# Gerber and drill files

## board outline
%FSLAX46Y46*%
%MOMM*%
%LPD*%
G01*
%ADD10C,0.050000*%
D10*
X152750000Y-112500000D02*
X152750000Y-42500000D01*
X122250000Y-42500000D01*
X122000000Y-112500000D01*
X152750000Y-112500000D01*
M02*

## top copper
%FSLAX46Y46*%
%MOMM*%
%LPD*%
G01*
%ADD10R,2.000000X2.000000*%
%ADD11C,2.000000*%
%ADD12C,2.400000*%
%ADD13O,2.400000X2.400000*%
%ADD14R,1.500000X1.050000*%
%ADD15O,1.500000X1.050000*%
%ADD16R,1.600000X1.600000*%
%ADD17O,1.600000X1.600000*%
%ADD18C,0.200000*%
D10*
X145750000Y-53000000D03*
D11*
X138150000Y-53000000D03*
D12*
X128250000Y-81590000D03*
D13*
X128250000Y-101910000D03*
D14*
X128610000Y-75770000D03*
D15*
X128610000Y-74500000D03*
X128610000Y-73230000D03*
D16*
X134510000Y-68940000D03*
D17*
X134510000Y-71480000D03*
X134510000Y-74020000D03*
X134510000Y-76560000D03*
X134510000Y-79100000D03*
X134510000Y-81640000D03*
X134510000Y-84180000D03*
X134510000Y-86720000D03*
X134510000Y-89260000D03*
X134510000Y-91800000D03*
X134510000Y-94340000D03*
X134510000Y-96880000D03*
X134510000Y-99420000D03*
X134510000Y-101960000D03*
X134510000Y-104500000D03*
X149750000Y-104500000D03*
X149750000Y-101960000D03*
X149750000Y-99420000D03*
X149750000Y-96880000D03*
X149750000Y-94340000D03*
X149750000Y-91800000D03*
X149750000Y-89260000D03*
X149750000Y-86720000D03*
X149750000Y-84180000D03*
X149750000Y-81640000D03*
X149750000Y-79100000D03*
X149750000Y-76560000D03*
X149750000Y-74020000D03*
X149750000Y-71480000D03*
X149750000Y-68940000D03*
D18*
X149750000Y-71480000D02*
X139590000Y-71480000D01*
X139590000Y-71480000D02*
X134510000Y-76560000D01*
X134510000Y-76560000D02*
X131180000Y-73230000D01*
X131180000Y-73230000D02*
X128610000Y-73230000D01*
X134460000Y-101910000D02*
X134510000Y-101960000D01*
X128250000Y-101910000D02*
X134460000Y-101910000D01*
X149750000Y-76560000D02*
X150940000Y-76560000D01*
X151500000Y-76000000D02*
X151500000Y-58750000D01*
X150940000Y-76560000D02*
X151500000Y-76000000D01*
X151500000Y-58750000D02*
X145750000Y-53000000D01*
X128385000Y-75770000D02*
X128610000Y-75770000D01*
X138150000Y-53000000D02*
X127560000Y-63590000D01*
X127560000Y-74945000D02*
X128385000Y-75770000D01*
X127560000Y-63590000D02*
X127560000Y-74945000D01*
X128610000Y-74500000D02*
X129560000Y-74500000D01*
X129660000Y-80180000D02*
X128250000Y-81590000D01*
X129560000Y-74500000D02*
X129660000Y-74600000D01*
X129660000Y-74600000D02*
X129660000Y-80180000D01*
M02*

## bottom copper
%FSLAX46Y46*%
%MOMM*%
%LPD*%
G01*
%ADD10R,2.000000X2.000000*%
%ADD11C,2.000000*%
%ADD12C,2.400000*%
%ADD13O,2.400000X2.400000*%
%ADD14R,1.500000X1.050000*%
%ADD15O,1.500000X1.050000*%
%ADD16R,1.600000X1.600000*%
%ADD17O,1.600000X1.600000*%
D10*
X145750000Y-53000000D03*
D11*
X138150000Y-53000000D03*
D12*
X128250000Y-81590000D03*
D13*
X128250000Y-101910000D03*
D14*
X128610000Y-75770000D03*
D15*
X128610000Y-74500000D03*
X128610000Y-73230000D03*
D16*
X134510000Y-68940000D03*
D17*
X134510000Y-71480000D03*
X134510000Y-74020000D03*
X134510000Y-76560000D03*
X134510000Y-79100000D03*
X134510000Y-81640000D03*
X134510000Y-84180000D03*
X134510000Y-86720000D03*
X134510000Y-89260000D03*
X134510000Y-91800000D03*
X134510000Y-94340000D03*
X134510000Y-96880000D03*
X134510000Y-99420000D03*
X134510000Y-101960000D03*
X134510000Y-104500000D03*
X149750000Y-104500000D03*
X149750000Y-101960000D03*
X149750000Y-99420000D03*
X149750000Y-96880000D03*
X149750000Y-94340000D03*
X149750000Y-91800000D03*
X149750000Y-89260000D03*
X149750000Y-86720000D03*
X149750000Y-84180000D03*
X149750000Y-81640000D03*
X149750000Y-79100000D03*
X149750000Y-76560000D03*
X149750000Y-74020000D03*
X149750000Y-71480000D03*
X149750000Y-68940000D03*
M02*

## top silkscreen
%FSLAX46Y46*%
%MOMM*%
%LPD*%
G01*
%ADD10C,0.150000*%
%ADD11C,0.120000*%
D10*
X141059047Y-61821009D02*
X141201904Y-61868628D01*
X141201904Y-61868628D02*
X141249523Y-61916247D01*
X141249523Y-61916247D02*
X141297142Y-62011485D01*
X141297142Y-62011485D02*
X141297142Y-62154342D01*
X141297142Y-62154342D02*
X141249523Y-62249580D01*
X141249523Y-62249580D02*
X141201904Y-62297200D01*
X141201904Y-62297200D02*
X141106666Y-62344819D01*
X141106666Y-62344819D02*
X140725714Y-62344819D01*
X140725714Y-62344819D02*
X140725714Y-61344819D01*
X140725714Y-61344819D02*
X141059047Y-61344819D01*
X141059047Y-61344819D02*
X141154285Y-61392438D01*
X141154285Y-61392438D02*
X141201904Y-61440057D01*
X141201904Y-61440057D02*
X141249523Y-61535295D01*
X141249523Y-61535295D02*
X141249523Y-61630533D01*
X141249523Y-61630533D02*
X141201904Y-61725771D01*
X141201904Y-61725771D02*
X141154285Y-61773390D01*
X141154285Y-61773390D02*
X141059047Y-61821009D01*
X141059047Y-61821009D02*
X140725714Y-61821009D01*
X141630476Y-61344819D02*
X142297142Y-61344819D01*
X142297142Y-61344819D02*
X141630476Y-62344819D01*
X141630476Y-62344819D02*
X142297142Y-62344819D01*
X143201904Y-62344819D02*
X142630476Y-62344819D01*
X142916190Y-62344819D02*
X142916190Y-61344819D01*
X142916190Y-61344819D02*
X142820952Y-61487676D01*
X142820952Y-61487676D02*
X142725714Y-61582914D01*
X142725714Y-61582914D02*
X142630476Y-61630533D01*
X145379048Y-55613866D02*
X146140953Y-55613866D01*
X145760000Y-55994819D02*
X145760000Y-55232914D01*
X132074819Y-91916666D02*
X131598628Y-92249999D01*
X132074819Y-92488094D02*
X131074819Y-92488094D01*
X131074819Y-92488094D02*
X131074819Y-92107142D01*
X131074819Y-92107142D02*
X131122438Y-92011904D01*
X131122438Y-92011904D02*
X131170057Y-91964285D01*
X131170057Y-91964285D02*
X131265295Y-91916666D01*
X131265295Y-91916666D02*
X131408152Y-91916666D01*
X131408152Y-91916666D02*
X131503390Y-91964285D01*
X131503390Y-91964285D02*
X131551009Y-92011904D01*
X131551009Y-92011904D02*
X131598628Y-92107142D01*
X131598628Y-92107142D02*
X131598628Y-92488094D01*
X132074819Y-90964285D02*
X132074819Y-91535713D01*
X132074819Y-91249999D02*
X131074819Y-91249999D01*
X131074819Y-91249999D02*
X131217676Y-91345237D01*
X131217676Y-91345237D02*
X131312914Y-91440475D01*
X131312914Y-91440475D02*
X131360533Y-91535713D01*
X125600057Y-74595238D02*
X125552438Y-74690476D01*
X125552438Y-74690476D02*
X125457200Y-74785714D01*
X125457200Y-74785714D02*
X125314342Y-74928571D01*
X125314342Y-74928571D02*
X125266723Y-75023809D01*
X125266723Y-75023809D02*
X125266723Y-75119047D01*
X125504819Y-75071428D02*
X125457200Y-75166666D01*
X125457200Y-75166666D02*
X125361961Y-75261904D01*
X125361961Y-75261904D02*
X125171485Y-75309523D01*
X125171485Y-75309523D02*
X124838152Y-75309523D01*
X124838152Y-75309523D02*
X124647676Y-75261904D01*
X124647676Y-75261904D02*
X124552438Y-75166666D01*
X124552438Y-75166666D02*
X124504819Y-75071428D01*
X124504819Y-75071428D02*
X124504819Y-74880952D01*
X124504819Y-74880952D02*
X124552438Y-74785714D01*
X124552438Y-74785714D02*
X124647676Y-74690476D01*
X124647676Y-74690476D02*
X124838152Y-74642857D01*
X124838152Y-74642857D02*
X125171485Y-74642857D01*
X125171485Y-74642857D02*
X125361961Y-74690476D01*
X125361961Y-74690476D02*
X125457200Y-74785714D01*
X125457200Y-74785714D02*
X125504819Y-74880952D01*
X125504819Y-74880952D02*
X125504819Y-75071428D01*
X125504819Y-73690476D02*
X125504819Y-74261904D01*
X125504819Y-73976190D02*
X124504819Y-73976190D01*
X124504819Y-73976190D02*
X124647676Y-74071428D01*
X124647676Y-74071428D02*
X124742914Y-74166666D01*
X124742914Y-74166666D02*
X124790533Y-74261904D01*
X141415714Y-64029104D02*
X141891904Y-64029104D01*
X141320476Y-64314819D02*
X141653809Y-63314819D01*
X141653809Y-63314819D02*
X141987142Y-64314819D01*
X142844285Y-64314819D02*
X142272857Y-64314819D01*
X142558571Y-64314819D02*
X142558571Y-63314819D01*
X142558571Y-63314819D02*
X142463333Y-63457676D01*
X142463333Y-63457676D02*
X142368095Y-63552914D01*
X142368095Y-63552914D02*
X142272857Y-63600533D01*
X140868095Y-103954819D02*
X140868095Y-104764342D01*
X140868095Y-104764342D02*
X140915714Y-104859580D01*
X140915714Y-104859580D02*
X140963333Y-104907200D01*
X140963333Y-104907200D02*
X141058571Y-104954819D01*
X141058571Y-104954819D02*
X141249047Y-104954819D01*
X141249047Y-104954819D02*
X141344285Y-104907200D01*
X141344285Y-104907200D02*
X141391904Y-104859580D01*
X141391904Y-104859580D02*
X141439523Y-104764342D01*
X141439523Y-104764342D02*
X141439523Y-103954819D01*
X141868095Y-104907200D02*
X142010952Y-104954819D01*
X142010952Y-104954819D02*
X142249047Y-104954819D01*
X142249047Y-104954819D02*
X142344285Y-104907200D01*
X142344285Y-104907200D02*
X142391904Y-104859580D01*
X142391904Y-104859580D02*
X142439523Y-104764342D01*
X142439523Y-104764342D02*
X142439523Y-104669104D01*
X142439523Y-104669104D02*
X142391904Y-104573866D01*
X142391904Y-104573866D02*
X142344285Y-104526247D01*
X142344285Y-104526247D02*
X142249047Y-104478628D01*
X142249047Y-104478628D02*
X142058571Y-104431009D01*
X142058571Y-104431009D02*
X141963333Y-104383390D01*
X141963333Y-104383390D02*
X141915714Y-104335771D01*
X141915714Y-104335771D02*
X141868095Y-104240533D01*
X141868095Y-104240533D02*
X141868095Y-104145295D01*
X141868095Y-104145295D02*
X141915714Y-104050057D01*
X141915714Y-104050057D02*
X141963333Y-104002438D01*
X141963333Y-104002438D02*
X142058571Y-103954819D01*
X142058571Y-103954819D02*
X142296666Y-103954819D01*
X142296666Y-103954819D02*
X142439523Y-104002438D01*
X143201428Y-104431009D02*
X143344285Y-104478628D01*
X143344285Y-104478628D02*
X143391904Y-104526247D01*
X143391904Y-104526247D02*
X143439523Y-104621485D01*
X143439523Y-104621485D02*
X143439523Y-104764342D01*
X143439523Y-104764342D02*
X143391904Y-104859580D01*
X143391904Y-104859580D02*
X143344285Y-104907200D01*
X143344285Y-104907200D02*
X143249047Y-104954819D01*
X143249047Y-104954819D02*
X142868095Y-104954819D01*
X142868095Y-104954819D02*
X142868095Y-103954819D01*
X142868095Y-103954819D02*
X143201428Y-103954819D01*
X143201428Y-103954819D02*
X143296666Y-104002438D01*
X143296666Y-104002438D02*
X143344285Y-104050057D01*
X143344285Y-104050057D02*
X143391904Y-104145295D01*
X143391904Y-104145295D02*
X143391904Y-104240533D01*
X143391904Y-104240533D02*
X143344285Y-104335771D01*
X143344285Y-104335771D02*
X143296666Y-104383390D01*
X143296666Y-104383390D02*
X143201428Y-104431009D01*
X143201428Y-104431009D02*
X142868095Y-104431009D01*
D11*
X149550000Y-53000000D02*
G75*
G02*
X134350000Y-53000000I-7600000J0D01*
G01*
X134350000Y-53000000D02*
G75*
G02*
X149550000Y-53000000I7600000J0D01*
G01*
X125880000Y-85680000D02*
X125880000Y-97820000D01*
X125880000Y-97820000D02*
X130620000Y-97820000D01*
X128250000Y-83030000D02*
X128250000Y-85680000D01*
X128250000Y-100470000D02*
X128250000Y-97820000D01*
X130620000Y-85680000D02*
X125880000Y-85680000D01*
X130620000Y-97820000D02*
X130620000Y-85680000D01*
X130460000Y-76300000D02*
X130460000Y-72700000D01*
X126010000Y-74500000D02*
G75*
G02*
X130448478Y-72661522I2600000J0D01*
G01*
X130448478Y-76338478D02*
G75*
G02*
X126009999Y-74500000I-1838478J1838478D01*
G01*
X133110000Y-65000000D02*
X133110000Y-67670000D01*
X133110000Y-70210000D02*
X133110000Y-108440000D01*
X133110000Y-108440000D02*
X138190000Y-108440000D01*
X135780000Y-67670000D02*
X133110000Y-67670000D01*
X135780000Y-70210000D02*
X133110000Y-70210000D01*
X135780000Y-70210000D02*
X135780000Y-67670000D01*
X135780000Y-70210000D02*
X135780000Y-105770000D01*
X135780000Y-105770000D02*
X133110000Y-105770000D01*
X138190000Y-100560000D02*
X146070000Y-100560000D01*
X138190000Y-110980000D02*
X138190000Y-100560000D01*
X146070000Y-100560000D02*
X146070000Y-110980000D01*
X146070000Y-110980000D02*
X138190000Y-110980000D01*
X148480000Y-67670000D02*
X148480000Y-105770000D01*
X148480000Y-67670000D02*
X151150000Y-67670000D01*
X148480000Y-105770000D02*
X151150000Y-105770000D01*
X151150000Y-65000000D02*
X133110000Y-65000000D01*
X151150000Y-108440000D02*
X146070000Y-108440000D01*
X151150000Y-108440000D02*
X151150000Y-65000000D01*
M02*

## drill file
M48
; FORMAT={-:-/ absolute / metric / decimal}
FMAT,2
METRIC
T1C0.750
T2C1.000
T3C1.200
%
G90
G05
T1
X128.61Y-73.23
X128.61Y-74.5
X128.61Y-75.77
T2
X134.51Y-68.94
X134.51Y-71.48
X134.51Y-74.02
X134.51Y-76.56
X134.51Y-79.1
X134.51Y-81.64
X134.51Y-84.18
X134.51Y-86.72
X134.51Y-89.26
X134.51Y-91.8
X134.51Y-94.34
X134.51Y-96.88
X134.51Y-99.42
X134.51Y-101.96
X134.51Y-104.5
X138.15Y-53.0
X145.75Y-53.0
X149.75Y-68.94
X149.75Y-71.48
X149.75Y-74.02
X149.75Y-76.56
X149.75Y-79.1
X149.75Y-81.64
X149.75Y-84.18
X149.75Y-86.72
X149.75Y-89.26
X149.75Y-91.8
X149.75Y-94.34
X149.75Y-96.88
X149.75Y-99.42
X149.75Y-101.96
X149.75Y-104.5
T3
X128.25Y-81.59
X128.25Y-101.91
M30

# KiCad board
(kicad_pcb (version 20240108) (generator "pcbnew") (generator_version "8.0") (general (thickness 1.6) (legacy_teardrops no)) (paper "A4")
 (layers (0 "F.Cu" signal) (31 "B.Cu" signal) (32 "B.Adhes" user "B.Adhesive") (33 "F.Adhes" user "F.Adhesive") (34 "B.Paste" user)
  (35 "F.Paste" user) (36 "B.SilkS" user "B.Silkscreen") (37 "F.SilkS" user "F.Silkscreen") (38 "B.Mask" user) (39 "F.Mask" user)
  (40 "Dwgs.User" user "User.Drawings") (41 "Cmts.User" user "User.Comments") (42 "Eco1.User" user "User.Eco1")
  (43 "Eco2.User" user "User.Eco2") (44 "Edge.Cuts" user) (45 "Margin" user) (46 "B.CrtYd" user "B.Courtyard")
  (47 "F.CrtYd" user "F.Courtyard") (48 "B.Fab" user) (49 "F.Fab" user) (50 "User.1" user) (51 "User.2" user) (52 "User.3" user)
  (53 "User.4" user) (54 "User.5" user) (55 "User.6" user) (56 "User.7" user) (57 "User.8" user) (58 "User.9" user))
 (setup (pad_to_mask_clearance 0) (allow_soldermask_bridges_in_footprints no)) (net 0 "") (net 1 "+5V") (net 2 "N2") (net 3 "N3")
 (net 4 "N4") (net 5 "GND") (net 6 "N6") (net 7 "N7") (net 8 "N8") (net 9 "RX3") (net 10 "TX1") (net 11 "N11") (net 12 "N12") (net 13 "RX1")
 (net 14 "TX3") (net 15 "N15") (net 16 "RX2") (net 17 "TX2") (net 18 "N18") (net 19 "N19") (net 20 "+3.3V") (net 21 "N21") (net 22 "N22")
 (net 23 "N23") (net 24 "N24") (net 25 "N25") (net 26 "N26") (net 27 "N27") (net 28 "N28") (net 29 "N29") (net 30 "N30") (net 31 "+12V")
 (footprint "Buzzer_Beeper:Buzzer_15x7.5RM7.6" (layer "F.Cu") (at 145.75 53 180)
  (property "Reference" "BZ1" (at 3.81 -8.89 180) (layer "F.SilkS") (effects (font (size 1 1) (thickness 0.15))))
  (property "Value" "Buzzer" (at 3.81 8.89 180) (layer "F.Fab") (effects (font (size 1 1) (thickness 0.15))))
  (fp_circle (center 3.8 0) (end 11.4 0) (stroke (width 0.12) (type solid)) (fill none) (layer "F.SilkS"))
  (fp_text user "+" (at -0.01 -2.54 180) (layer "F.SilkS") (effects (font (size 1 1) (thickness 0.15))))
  (pad "1" thru_hole rect (at 0 0 180) (size 2 2) (drill 1) (layers "*.Cu" "*.Mask") (remove_unused_layers no) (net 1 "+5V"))
  (pad "2" thru_hole circle (at 7.6 0 180) (size 2 2) (drill 1) (layers "*.Cu" "*.Mask") (remove_unused_layers no) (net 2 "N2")))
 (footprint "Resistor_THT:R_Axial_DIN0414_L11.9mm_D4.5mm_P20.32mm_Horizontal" (layer "F.Cu") (at 128.25 81.59 -90)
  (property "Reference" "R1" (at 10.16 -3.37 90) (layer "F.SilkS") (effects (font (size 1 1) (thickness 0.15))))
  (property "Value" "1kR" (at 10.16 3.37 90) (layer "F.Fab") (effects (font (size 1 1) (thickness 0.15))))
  (fp_line (start 4.09 2.37) (end 16.23 2.37) (stroke (width 0.12) (type solid)) (layer "F.SilkS"))
  (fp_line (start 16.23 2.37) (end 16.23 -2.37) (stroke (width 0.12) (type solid)) (layer "F.SilkS"))
  (fp_line (start 1.44 0) (end 4.09 0) (stroke (width 0.12) (type solid)) (layer "F.SilkS"))
  (fp_line (start 18.88 0) (end 16.23 0) (stroke (width 0.12) (type solid)) (layer "F.SilkS"))
  (fp_line (start 4.09 -2.37) (end 4.09 2.37) (stroke (width 0.12) (type solid)) (layer "F.SilkS"))
  (fp_line (start 16.23 -2.37) (end 4.09 -2.37) (stroke (width 0.12) (type solid)) (layer "F.SilkS"))
  (pad "1" thru_hole circle (at 0 0 270) (size 2.4 2.4) (drill 1.2) (layers "*.Cu" "*.Mask") (remove_unused_layers no) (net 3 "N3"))
  (pad "2" thru_hole oval (at 20.32 0 270) (size 2.4 2.4) (drill 1.2) (layers "*.Cu" "*.Mask") (remove_unused_layers no) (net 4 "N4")))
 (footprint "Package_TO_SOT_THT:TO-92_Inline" (layer "F.Cu") (at 128.61 75.77 90)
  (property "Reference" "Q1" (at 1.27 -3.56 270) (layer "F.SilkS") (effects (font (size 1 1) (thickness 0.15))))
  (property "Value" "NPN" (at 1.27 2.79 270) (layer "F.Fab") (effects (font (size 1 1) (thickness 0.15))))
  (fp_line (start -0.53 1.85) (end 3.07 1.85) (stroke (width 0.12) (type solid)) (layer "F.SilkS"))
  (fp_arc (start 1.27 -2.6) (mid 3.672087 -0.994977) (end 3.108478 1.838478) (stroke (width 0.12) (type solid)) (layer "F.SilkS"))
  (fp_arc (start -0.568478 1.838478) (mid -1.132087 -0.994977) (end 1.27 -2.6) (stroke (width 0.12) (type solid)) (layer "F.SilkS"))
  (pad "1" thru_hole rect (at 0 0 90) (size 1.05 1.5) (drill 0.75) (layers "*.Cu" "*.Mask") (remove_unused_layers no) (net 2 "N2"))
  (pad "2" thru_hole oval (at 1.27 0 90) (size 1.05 1.5) (drill 0.75) (layers "*.Cu" "*.Mask") (remove_unused_layers no) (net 3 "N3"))
  (pad "3" thru_hole oval (at 2.54 0 90) (size 1.05 1.5) (drill 0.75) (layers "*.Cu" "*.Mask") (remove_unused_layers no) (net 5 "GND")))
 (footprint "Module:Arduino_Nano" (layer "F.Cu") (at 134.51 68.94)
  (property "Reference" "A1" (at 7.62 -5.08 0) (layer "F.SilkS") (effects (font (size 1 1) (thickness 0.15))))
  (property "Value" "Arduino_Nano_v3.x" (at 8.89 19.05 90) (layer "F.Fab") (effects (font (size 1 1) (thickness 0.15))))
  (fp_line (start -1.4 -3.94) (end -1.4 -1.27) (stroke (width 0.12) (type solid)) (layer "F.SilkS"))
  (fp_line (start -1.4 1.27) (end -1.4 39.5) (stroke (width 0.12) (type solid)) (layer "F.SilkS"))
  (fp_line (start -1.4 39.5) (end 3.68 39.5) (stroke (width 0.12) (type solid)) (layer "F.SilkS"))
  (fp_line (start 1.27 -1.27) (end -1.4 -1.27) (stroke (width 0.12) (type solid)) (layer "F.SilkS"))
  (fp_line (start 1.27 1.27) (end -1.4 1.27) (stroke (width 0.12) (type solid)) (layer "F.SilkS"))
  (fp_line (start 1.27 1.27) (end 1.27 -1.27) (stroke (width 0.12) (type solid)) (layer "F.SilkS"))
  (fp_line (start 1.27 1.27) (end 1.27 36.83) (stroke (width 0.12) (type solid)) (layer "F.SilkS"))
  (fp_line (start 1.27 36.83) (end -1.4 36.83) (stroke (width 0.12) (type solid)) (layer "F.SilkS"))
  (fp_line (start 3.68 31.62) (end 11.56 31.62) (stroke (width 0.12) (type solid)) (layer "F.SilkS"))
  (fp_line (start 3.68 42.04) (end 3.68 31.62) (stroke (width 0.12) (type solid)) (layer "F.SilkS"))
  (fp_line (start 11.56 31.62) (end 11.56 42.04) (stroke (width 0.12) (type solid)) (layer "F.SilkS"))
  (fp_line (start 11.56 42.04) (end 3.68 42.04) (stroke (width 0.12) (type solid)) (layer "F.SilkS"))
  (fp_line (start 13.97 -1.27) (end 13.97 36.83) (stroke (width 0.12) (type solid)) (layer "F.SilkS"))
  (fp_line (start 13.97 -1.27) (end 16.64 -1.27) (stroke (width 0.12) (type solid)) (layer "F.SilkS"))
  (fp_line (start 13.97 36.83) (end 16.64 36.83) (stroke (width 0.12) (type solid)) (layer "F.SilkS"))
  (fp_line (start 16.64 -3.94) (end -1.4 -3.94) (stroke (width 0.12) (type solid)) (layer "F.SilkS"))
  (fp_line (start 16.64 39.5) (end 11.56 39.5) (stroke (width 0.12) (type solid)) (layer "F.SilkS"))
  (fp_line (start 16.64 39.5) (end 16.64 -3.94) (stroke (width 0.12) (type solid)) (layer "F.SilkS"))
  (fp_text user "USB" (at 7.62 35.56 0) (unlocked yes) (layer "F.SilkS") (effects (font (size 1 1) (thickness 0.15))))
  (pad "1" thru_hole rect (at 0 0) (size 1.6 1.6) (drill 1) (layers "*.Cu" "*.Mask") (remove_unused_layers no) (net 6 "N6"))
  (pad "2" thru_hole oval (at 0 2.54) (size 1.6 1.6) (drill 1) (layers "*.Cu" "*.Mask") (remove_unused_layers no) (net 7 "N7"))
  (pad "3" thru_hole oval (at 0 5.08) (size 1.6 1.6) (drill 1) (layers "*.Cu" "*.Mask") (remove_unused_layers no) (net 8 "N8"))
  (pad "4" thru_hole oval (at 0 7.62) (size 1.6 1.6) (drill 1) (layers "*.Cu" "*.Mask") (remove_unused_layers no) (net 5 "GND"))
  (pad "5" thru_hole oval (at 0 10.16) (size 1.6 1.6) (drill 1) (layers "*.Cu" "*.Mask") (remove_unused_layers no) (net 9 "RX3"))
  (pad "6" thru_hole oval (at 0 12.7) (size 1.6 1.6) (drill 1) (layers "*.Cu" "*.Mask") (remove_unused_layers no) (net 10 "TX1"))
  (pad "7" thru_hole oval (at 0 15.24) (size 1.6 1.6) (drill 1) (layers "*.Cu" "*.Mask") (remove_unused_layers no) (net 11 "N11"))
  (pad "8" thru_hole oval (at 0 17.78) (size 1.6 1.6) (drill 1) (layers "*.Cu" "*.Mask") (remove_unused_layers no) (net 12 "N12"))
  (pad "9" thru_hole oval (at 0 20.32) (size 1.6 1.6) (drill 1) (layers "*.Cu" "*.Mask") (remove_unused_layers no) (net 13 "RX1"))
  (pad "10" thru_hole oval (at 0 22.86) (size 1.6 1.6) (drill 1) (layers "*.Cu" "*.Mask") (remove_unused_layers no) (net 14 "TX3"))
  (pad "11" thru_hole oval (at 0 25.4) (size 1.6 1.6) (drill 1) (layers "*.Cu" "*.Mask") (remove_unused_layers no) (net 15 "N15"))
  (pad "12" thru_hole oval (at 0 27.94) (size 1.6 1.6) (drill 1) (layers "*.Cu" "*.Mask") (remove_unused_layers no) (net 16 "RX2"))
  (pad "13" thru_hole oval (at 0 30.48) (size 1.6 1.6) (drill 1) (layers "*.Cu" "*.Mask") (remove_unused_layers no) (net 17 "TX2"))
  (pad "14" thru_hole oval (at 0 33.02) (size 1.6 1.6) (drill 1) (layers "*.Cu" "*.Mask") (remove_unused_layers no) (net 4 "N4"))
  (pad "15" thru_hole oval (at 0 35.56) (size 1.6 1.6) (drill 1) (layers "*.Cu" "*.Mask") (remove_unused_layers no) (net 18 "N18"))
  (pad "16" thru_hole oval (at 15.24 35.56) (size 1.6 1.6) (drill 1) (layers "*.Cu" "*.Mask") (remove_unused_layers no) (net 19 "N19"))
  (pad "17" thru_hole oval (at 15.24 33.02) (size 1.6 1.6) (drill 1) (layers "*.Cu" "*.Mask") (remove_unused_layers no) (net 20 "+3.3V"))
  (pad "18" thru_hole oval (at 15.24 30.48) (size 1.6 1.6) (drill 1) (layers "*.Cu" "*.Mask") (remove_unused_layers no) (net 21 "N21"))
  (pad "19" thru_hole oval (at 15.24 27.94) (size 1.6 1.6) (drill 1) (layers "*.Cu" "*.Mask") (remove_unused_layers no) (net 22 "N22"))
  (pad "20" thru_hole oval (at 15.24 25.4) (size 1.6 1.6) (drill 1) (layers "*.Cu" "*.Mask") (remove_unused_layers no) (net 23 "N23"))
  (pad "21" thru_hole oval (at 15.24 22.86) (size 1.6 1.6) (drill 1) (layers "*.Cu" "*.Mask") (remove_unused_layers no) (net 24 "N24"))
  (pad "22" thru_hole oval (at 15.24 20.32) (size 1.6 1.6) (drill 1) (layers "*.Cu" "*.Mask") (remove_unused_layers no) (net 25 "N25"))
  (pad "23" thru_hole oval (at 15.24 17.78) (size 1.6 1.6) (drill 1) (layers "*.Cu" "*.Mask") (remove_unused_layers no) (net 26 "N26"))
  (pad "24" thru_hole oval (at 15.24 15.24) (size 1.6 1.6) (drill 1) (layers "*.Cu" "*.Mask") (remove_unused_layers no) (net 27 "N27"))
  (pad "25" thru_hole oval (at 15.24 12.7) (size 1.6 1.6) (drill 1) (layers "*.Cu" "*.Mask") (remove_unused_layers no) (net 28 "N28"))
  (pad "26" thru_hole oval (at 15.24 10.16) (size 1.6 1.6) (drill 1) (layers "*.Cu" "*.Mask") (remove_unused_layers no) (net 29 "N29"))
  (pad "27" thru_hole oval (at 15.24 7.62) (size 1.6 1.6) (drill 1) (layers "*.Cu" "*.Mask") (remove_unused_layers no) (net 1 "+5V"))
  (pad "28" thru_hole oval (at 15.24 5.08) (size 1.6 1.6) (drill 1) (layers "*.Cu" "*.Mask") (remove_unused_layers no) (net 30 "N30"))
  (pad "29" thru_hole oval (at 15.24 2.54) (size 1.6 1.6) (drill 1) (layers "*.Cu" "*.Mask") (remove_unused_layers no) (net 5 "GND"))
  (pad "30" thru_hole oval (at 15.24 0) (size 1.6 1.6) (drill 1) (layers "*.Cu" "*.Mask") (remove_unused_layers no) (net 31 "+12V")))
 (gr_poly
  (pts (xy 152.75 112.5) (xy 152.75 42.5) (xy 122.25 42.5) (xy 122 112.5)) (stroke (width 0.05) (type solid)) (fill none)
  (layer "Edge.Cuts"))
 (segment (start 149.75 71.48) (end 139.59 71.48) (width 0.2) (layer "F.Cu") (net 5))
 (segment (start 139.59 71.48) (end 134.51 76.56) (width 0.2) (layer "F.Cu") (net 5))
 (segment (start 134.51 76.56) (end 131.18 73.23) (width 0.2) (layer "F.Cu") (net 5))
 (segment (start 131.18 73.23) (end 128.61 73.23) (width 0.2) (layer "F.Cu") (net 5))
 (segment (start 134.46 101.91) (end 134.51 101.96) (width 0.2) (layer "F.Cu") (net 4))
 (segment (start 128.25 101.91) (end 134.46 101.91) (width 0.2) (layer "F.Cu") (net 4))
 (segment (start 149.75 76.56) (end 150.94 76.56) (width 0.2) (layer "F.Cu") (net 1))
 (segment (start 151.5 76) (end 151.5 58.75) (width 0.2) (layer "F.Cu") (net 1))
 (segment (start 150.94 76.56) (end 151.5 76) (width 0.2) (layer "F.Cu") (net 1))
 (segment (start 151.5 58.75) (end 145.75 53) (width 0.2) (layer "F.Cu") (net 1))
 (segment (start 128.385 75.77) (end 128.61 75.77) (width 0.2) (layer "F.Cu") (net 2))
 (segment (start 138.15 53) (end 127.56 63.59) (width 0.2) (layer "F.Cu") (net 2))
 (segment (start 127.56 74.945) (end 128.385 75.77) (width 0.2) (layer "F.Cu") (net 2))
 (segment (start 127.56 63.59) (end 127.56 74.945) (width 0.2) (layer "F.Cu") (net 2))
 (segment (start 128.61 74.5) (end 129.56 74.5) (width 0.2) (layer "F.Cu") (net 3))
 (segment (start 129.66 80.18) (end 128.25 81.59) (width 0.2) (layer "F.Cu") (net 3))
 (segment (start 129.56 74.5) (end 129.66 74.6) (width 0.2) (layer "F.Cu") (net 3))
 (segment (start 129.66 74.6) (end 129.66 80.18) (width 0.2) (layer "F.Cu") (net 3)))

